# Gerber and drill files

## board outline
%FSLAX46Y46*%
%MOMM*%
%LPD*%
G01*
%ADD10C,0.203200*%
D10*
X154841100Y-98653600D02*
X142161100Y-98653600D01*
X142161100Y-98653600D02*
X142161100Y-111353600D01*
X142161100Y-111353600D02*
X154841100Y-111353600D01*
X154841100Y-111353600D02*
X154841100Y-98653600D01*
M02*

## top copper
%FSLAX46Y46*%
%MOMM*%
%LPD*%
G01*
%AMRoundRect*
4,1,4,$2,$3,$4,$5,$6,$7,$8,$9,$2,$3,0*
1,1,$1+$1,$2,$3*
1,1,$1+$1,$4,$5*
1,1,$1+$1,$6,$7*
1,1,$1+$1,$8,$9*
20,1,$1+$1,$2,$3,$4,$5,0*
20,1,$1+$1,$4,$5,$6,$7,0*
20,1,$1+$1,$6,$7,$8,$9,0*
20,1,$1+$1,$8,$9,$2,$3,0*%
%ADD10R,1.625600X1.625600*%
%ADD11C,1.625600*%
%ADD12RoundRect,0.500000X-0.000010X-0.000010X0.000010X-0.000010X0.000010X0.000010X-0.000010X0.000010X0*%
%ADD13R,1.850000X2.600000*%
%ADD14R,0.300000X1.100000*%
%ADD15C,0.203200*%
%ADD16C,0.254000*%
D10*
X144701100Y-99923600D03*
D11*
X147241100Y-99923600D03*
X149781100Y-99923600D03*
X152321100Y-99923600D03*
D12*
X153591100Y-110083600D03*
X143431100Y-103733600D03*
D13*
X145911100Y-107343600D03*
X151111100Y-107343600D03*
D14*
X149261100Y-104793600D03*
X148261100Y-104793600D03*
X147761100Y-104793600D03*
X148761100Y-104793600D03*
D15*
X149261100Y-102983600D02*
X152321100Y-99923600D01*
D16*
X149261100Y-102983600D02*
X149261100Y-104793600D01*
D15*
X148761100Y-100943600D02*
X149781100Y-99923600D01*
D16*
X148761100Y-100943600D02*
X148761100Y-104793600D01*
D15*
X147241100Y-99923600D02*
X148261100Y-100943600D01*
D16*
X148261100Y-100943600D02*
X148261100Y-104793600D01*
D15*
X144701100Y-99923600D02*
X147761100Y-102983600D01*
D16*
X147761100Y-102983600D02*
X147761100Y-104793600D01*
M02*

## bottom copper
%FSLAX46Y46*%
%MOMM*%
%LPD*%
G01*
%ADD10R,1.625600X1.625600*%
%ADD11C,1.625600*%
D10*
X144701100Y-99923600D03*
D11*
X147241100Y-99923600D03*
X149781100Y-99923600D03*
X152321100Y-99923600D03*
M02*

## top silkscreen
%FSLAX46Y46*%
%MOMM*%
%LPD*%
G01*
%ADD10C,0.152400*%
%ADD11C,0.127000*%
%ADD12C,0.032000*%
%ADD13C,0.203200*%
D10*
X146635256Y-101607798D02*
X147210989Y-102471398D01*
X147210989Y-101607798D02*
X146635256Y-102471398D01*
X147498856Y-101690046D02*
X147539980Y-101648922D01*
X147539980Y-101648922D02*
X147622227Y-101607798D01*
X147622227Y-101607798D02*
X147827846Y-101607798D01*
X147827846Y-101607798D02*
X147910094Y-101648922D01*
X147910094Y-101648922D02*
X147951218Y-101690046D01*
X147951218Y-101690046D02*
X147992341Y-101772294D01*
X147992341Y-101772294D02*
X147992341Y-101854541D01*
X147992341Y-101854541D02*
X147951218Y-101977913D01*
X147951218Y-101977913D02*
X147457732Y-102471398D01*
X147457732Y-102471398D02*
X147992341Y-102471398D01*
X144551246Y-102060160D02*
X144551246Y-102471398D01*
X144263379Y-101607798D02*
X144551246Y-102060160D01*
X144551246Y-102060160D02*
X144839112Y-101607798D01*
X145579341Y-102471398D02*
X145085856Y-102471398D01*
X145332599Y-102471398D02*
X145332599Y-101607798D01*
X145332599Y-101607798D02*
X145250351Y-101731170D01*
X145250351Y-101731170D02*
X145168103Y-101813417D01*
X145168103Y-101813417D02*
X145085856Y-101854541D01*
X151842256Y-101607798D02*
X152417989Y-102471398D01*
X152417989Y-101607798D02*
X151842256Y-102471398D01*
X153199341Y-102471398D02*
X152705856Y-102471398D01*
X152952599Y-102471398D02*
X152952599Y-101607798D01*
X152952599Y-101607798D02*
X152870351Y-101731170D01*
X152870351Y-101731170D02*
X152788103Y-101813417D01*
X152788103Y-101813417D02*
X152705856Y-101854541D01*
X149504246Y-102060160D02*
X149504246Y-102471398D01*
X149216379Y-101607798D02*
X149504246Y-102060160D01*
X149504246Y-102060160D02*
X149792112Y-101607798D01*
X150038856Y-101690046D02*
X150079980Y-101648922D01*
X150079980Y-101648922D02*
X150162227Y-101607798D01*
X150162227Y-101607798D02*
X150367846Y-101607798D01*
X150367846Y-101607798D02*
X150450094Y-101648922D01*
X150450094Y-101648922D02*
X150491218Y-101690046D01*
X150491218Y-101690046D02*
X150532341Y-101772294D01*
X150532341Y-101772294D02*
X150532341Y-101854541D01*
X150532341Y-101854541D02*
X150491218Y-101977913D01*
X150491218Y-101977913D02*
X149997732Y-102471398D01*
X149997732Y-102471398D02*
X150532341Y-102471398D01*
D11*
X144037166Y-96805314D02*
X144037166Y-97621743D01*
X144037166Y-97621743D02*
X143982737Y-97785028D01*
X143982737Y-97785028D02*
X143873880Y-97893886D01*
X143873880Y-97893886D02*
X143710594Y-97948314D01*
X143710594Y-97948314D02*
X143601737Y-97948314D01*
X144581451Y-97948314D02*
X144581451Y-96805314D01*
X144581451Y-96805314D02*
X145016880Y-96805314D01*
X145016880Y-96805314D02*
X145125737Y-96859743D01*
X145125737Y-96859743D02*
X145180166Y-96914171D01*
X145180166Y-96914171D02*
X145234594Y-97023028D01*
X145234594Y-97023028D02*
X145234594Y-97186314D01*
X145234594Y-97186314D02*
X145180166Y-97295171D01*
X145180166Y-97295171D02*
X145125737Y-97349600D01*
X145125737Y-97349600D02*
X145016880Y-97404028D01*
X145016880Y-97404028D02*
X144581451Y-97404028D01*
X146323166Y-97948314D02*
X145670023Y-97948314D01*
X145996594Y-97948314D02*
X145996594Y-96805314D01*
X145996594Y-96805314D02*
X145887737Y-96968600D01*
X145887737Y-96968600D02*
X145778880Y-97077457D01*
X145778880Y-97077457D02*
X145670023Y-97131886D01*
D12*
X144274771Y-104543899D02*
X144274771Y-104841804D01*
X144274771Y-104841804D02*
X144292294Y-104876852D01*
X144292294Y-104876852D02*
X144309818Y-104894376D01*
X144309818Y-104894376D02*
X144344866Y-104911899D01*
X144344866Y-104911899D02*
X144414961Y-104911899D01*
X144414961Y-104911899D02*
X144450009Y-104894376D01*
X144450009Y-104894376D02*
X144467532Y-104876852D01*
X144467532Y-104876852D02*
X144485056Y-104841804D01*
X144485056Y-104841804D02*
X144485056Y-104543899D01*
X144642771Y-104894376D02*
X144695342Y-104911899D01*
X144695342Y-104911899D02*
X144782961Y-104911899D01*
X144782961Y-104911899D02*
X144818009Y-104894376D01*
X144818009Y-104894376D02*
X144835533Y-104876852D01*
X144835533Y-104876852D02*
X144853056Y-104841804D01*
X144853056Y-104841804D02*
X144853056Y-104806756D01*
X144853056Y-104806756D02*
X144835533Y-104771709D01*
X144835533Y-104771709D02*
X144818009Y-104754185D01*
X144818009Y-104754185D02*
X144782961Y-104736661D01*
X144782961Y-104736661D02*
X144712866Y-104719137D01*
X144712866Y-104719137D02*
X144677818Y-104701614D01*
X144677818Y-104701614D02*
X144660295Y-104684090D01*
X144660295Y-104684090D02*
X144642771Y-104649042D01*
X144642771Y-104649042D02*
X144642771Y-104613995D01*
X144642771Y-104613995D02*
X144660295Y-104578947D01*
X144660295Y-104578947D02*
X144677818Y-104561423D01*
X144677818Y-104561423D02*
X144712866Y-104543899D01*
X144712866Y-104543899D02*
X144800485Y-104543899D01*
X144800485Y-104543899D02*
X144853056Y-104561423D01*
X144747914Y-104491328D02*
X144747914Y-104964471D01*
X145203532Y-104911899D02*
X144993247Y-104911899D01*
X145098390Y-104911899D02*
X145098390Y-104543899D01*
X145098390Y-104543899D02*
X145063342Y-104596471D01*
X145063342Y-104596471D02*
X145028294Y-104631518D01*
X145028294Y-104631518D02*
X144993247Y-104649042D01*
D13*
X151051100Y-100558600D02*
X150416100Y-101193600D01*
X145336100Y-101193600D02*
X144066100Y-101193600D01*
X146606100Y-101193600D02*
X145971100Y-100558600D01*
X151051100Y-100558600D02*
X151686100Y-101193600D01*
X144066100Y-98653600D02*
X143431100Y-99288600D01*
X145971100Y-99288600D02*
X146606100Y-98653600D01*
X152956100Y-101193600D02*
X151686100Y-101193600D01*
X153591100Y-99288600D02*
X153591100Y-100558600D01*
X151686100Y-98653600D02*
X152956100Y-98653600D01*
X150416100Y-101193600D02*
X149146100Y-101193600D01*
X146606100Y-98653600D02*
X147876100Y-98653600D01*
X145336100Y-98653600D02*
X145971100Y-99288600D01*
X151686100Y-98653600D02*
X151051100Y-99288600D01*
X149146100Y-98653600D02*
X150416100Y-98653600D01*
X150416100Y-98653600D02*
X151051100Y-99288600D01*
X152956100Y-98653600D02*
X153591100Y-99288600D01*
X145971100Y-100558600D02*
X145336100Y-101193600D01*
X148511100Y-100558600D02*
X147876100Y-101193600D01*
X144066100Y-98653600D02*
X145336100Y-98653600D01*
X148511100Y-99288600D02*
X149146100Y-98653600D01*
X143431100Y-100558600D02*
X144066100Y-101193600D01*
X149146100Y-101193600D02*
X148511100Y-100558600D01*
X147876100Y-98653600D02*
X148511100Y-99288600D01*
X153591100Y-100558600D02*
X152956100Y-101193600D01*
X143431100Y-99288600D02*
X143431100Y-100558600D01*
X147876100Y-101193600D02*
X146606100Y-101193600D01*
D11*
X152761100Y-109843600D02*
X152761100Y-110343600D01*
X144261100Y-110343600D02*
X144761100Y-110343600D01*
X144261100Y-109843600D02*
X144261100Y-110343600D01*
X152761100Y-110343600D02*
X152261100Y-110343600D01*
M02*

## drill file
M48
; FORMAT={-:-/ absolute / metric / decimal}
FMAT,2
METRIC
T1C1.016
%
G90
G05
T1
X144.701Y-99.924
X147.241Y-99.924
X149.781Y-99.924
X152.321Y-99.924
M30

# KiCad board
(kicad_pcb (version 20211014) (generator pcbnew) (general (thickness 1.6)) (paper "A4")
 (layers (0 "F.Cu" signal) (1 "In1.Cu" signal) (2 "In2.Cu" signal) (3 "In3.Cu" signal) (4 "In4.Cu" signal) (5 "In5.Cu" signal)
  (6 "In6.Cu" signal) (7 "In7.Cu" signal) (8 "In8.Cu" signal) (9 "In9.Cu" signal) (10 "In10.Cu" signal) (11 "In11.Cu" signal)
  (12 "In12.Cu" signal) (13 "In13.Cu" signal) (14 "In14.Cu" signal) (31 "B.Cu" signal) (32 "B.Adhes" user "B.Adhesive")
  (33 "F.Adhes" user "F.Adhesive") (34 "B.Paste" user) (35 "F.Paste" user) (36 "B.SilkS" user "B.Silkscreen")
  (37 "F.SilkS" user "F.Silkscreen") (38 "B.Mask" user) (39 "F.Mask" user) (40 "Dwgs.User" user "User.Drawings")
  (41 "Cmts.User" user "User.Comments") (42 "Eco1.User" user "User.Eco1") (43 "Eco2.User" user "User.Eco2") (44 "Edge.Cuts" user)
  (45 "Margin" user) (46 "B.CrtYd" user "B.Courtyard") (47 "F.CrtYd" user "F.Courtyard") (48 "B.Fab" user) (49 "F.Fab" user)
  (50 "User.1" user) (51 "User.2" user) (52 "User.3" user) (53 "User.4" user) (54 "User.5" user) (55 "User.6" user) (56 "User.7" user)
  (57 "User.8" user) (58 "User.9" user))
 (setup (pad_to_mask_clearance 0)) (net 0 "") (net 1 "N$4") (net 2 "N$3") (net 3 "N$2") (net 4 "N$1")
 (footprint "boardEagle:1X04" (layer "F.Cu") (at 144.7011 99.9236)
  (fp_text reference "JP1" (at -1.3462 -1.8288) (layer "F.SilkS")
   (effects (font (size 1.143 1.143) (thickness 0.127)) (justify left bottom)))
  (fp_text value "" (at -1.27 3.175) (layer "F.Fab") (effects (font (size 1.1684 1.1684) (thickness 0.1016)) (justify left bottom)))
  (fp_line (start 6.35 0.635) (end 5.715 1.27) (layer "F.SilkS") (width 0.2032))
  (fp_line (start 0.635 1.27) (end -0.635 1.27) (layer "F.SilkS") (width 0.2032))
  (fp_line (start 1.905 1.27) (end 1.27 0.635) (layer "F.SilkS") (width 0.2032))
  (fp_line (start 6.35 0.635) (end 6.985 1.27) (layer "F.SilkS") (width 0.2032))
  (fp_line (start -0.635 -1.27) (end -1.27 -0.635) (layer "F.SilkS") (width 0.2032))
  (fp_line (start 1.27 -0.635) (end 1.905 -1.27) (layer "F.SilkS") (width 0.2032))
  (fp_line (start 8.255 1.27) (end 6.985 1.27) (layer "F.SilkS") (width 0.2032))
  (fp_line (start 8.89 -0.635) (end 8.89 0.635) (layer "F.SilkS") (width 0.2032))
  (fp_line (start 6.985 -1.27) (end 8.255 -1.27) (layer "F.SilkS") (width 0.2032))
  (fp_line (start 5.715 1.27) (end 4.445 1.27) (layer "F.SilkS") (width 0.2032))
  (fp_line (start 1.905 -1.27) (end 3.175 -1.27) (layer "F.SilkS") (width 0.2032))
  (fp_line (start 0.635 -1.27) (end 1.27 -0.635) (layer "F.SilkS") (width 0.2032))
  (fp_line (start 6.985 -1.27) (end 6.35 -0.635) (layer "F.SilkS") (width 0.2032))
  (fp_line (start 4.445 -1.27) (end 5.715 -1.27) (layer "F.SilkS") (width 0.2032))
  (fp_line (start 5.715 -1.27) (end 6.35 -0.635) (layer "F.SilkS") (width 0.2032))
  (fp_line (start 8.255 -1.27) (end 8.89 -0.635) (layer "F.SilkS") (width 0.2032))
  (fp_line (start 1.27 0.635) (end 0.635 1.27) (layer "F.SilkS") (width 0.2032))
  (fp_line (start 3.81 0.635) (end 3.175 1.27) (layer "F.SilkS") (width 0.2032))
  (fp_line (start -0.635 -1.27) (end 0.635 -1.27) (layer "F.SilkS") (width 0.2032))
  (fp_line (start 3.81 -0.635) (end 4.445 -1.27) (layer "F.SilkS") (width 0.2032))
  (fp_line (start -1.27 0.635) (end -0.635 1.27) (layer "F.SilkS") (width 0.2032))
  (fp_line (start 4.445 1.27) (end 3.81 0.635) (layer "F.SilkS") (width 0.2032))
  (fp_line (start 3.175 -1.27) (end 3.81 -0.635) (layer "F.SilkS") (width 0.2032))
  (fp_line (start 8.89 0.635) (end 8.255 1.27) (layer "F.SilkS") (width 0.2032))
  (fp_line (start -1.27 -0.635) (end -1.27 0.635) (layer "F.SilkS") (width 0.2032))
  (fp_line (start 3.175 1.27) (end 1.905 1.27) (layer "F.SilkS") (width 0.2032))
  (pad "1" thru_hole rect (at 0 0 90) (size 1.6256 1.6256) (drill 1.016) (layers *.Cu *.Mask) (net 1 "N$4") (solder_mask_margin 0.1016))
  (pad "2" thru_hole circle (at 2.54 0 90) (size 1.6256 1.6256) (drill 1.016) (layers *.Cu *.Mask) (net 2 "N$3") (solder_mask_margin 0.1016))
  (pad "3" thru_hole circle (at 5.08 0 90) (size 1.6256 1.6256) (drill 1.016) (layers *.Cu *.Mask) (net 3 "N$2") (solder_mask_margin 0.1016))
  (pad "4" thru_hole circle (at 7.62 0 90) (size 1.6256 1.6256) (drill 1.016) (layers *.Cu *.Mask) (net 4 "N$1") (solder_mask_margin 0.1016)))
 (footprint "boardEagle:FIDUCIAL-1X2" (layer "F.Cu") (at 153.5911 110.0836)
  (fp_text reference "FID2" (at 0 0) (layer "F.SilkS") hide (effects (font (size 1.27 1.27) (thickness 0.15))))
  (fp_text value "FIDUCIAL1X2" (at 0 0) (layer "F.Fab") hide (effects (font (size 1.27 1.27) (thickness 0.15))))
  (pad "1" smd roundrect (at 0 0) (size 1 1) (layers "F.Cu" "F.Mask") (roundrect_rratio 0.5) (solder_mask_margin 0.1016)))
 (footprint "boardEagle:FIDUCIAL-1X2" (layer "F.Cu") (at 143.4311 103.7336)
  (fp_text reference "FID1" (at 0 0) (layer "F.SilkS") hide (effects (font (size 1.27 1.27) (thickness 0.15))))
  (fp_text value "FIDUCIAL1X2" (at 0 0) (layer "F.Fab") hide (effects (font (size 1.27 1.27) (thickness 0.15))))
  (pad "1" smd roundrect (at 0 0) (size 1 1) (layers "F.Cu" "F.Mask") (roundrect_rratio 0.5) (solder_mask_margin 0.1016)))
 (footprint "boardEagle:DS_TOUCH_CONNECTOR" (layer "F.Cu") (at 148.5111 107.5436)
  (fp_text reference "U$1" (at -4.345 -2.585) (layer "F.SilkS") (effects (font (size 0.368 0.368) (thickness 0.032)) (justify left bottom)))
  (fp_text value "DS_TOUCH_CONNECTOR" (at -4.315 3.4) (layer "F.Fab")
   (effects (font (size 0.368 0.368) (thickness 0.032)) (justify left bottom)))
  (fp_line (start 4.25 2.3) (end 4.25 2.8) (layer "F.SilkS") (width 0.127))
  (fp_line (start -4.25 2.8) (end -3.75 2.8) (layer "F.SilkS") (width 0.127))
  (fp_line (start -4.25 2.3) (end -4.25 2.8) (layer "F.SilkS") (width 0.127))
  (fp_line (start 4.25 2.8) (end 3.75 2.8) (layer "F.SilkS") (width 0.127))
  (pad "P$5" smd rect (at -2.6 -0.2) (size 1.85 2.6) (layers "F.Cu" "F.Paste" "F.Mask") (solder_mask_margin 0.1016))
  (pad "P$6" smd rect (at 2.6 -0.2) (size 1.85 2.6) (layers "F.Cu" "F.Paste" "F.Mask") (solder_mask_margin 0.1016))
  (pad "X1" smd rect (at 0.75 -2.75 90) (size 1.1 0.3) (layers "F.Cu" "F.Paste" "F.Mask") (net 4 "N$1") (solder_mask_margin 0.1016))
  (pad "X2" smd rect (at -0.25 -2.75 90) (size 1.1 0.3) (layers "F.Cu" "F.Paste" "F.Mask") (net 2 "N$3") (solder_mask_margin 0.1016))
  (pad "Y1" smd rect (at -0.75 -2.75 90) (size 1.1 0.3) (layers "F.Cu" "F.Paste" "F.Mask") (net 1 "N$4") (solder_mask_margin 0.1016))
  (pad "Y2" smd rect (at 0.25 -2.75 90) (size 1.1 0.3) (layers "F.Cu" "F.Paste" "F.Mask") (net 3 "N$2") (solder_mask_margin 0.1016)))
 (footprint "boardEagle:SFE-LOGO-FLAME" (layer "B.Cu") (at 149.6541 104.2416 -90)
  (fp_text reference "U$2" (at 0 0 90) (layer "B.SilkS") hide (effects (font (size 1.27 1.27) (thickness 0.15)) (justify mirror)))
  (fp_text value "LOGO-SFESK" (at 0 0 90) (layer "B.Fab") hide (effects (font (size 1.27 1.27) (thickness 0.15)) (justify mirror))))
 (gr_line (start 154.8411 98.6536) (end 142.1611 98.6536) (layer "Edge.Cuts") (width 0.2032))
 (gr_line (start 142.1611 98.6536) (end 142.1611 111.3536) (layer "Edge.Cuts") (width 0.2032))
 (gr_line (start 142.1611 111.3536) (end 154.8411 111.3536) (layer "Edge.Cuts") (width 0.2032))
 (gr_line (start 154.8411 111.3536) (end 154.8411 98.6536) (layer "Edge.Cuts") (width 0.2032))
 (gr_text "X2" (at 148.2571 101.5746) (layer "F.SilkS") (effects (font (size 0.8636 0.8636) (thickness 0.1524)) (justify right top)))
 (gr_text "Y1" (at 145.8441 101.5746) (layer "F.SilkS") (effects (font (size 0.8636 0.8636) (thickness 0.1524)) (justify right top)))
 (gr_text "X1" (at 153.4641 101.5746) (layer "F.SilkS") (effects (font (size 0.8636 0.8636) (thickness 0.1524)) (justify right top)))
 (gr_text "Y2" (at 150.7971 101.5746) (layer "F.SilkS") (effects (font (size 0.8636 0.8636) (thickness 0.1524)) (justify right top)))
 (segment (start 149.2611 102.9836) (end 152.3211 99.9236) (width 0.2032) (layer "F.Cu") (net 4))
 (segment (start 149.2611 102.9836) (end 149.2611 104.7936) (width 0.254) (layer "F.Cu") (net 4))
 (segment (start 148.7611 100.9436) (end 149.7811 99.9236) (width 0.2032) (layer "F.Cu") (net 3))
 (segment (start 148.7611 100.9436) (end 148.7611 104.7936) (width 0.254) (layer "F.Cu") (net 3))
 (segment (start 147.2411 99.9236) (end 148.2611 100.9436) (width 0.2032) (layer "F.Cu") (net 2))
 (segment (start 148.2611 100.9436) (end 148.2611 104.7936) (width 0.254) (layer "F.Cu") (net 2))
 (segment (start 144.7011 99.9236) (end 147.7611 102.9836) (width 0.2032) (layer "F.Cu") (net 1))
 (segment (start 147.7611 102.9836) (end 147.7611 104.7936) (width 0.254) (layer "F.Cu") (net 1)))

